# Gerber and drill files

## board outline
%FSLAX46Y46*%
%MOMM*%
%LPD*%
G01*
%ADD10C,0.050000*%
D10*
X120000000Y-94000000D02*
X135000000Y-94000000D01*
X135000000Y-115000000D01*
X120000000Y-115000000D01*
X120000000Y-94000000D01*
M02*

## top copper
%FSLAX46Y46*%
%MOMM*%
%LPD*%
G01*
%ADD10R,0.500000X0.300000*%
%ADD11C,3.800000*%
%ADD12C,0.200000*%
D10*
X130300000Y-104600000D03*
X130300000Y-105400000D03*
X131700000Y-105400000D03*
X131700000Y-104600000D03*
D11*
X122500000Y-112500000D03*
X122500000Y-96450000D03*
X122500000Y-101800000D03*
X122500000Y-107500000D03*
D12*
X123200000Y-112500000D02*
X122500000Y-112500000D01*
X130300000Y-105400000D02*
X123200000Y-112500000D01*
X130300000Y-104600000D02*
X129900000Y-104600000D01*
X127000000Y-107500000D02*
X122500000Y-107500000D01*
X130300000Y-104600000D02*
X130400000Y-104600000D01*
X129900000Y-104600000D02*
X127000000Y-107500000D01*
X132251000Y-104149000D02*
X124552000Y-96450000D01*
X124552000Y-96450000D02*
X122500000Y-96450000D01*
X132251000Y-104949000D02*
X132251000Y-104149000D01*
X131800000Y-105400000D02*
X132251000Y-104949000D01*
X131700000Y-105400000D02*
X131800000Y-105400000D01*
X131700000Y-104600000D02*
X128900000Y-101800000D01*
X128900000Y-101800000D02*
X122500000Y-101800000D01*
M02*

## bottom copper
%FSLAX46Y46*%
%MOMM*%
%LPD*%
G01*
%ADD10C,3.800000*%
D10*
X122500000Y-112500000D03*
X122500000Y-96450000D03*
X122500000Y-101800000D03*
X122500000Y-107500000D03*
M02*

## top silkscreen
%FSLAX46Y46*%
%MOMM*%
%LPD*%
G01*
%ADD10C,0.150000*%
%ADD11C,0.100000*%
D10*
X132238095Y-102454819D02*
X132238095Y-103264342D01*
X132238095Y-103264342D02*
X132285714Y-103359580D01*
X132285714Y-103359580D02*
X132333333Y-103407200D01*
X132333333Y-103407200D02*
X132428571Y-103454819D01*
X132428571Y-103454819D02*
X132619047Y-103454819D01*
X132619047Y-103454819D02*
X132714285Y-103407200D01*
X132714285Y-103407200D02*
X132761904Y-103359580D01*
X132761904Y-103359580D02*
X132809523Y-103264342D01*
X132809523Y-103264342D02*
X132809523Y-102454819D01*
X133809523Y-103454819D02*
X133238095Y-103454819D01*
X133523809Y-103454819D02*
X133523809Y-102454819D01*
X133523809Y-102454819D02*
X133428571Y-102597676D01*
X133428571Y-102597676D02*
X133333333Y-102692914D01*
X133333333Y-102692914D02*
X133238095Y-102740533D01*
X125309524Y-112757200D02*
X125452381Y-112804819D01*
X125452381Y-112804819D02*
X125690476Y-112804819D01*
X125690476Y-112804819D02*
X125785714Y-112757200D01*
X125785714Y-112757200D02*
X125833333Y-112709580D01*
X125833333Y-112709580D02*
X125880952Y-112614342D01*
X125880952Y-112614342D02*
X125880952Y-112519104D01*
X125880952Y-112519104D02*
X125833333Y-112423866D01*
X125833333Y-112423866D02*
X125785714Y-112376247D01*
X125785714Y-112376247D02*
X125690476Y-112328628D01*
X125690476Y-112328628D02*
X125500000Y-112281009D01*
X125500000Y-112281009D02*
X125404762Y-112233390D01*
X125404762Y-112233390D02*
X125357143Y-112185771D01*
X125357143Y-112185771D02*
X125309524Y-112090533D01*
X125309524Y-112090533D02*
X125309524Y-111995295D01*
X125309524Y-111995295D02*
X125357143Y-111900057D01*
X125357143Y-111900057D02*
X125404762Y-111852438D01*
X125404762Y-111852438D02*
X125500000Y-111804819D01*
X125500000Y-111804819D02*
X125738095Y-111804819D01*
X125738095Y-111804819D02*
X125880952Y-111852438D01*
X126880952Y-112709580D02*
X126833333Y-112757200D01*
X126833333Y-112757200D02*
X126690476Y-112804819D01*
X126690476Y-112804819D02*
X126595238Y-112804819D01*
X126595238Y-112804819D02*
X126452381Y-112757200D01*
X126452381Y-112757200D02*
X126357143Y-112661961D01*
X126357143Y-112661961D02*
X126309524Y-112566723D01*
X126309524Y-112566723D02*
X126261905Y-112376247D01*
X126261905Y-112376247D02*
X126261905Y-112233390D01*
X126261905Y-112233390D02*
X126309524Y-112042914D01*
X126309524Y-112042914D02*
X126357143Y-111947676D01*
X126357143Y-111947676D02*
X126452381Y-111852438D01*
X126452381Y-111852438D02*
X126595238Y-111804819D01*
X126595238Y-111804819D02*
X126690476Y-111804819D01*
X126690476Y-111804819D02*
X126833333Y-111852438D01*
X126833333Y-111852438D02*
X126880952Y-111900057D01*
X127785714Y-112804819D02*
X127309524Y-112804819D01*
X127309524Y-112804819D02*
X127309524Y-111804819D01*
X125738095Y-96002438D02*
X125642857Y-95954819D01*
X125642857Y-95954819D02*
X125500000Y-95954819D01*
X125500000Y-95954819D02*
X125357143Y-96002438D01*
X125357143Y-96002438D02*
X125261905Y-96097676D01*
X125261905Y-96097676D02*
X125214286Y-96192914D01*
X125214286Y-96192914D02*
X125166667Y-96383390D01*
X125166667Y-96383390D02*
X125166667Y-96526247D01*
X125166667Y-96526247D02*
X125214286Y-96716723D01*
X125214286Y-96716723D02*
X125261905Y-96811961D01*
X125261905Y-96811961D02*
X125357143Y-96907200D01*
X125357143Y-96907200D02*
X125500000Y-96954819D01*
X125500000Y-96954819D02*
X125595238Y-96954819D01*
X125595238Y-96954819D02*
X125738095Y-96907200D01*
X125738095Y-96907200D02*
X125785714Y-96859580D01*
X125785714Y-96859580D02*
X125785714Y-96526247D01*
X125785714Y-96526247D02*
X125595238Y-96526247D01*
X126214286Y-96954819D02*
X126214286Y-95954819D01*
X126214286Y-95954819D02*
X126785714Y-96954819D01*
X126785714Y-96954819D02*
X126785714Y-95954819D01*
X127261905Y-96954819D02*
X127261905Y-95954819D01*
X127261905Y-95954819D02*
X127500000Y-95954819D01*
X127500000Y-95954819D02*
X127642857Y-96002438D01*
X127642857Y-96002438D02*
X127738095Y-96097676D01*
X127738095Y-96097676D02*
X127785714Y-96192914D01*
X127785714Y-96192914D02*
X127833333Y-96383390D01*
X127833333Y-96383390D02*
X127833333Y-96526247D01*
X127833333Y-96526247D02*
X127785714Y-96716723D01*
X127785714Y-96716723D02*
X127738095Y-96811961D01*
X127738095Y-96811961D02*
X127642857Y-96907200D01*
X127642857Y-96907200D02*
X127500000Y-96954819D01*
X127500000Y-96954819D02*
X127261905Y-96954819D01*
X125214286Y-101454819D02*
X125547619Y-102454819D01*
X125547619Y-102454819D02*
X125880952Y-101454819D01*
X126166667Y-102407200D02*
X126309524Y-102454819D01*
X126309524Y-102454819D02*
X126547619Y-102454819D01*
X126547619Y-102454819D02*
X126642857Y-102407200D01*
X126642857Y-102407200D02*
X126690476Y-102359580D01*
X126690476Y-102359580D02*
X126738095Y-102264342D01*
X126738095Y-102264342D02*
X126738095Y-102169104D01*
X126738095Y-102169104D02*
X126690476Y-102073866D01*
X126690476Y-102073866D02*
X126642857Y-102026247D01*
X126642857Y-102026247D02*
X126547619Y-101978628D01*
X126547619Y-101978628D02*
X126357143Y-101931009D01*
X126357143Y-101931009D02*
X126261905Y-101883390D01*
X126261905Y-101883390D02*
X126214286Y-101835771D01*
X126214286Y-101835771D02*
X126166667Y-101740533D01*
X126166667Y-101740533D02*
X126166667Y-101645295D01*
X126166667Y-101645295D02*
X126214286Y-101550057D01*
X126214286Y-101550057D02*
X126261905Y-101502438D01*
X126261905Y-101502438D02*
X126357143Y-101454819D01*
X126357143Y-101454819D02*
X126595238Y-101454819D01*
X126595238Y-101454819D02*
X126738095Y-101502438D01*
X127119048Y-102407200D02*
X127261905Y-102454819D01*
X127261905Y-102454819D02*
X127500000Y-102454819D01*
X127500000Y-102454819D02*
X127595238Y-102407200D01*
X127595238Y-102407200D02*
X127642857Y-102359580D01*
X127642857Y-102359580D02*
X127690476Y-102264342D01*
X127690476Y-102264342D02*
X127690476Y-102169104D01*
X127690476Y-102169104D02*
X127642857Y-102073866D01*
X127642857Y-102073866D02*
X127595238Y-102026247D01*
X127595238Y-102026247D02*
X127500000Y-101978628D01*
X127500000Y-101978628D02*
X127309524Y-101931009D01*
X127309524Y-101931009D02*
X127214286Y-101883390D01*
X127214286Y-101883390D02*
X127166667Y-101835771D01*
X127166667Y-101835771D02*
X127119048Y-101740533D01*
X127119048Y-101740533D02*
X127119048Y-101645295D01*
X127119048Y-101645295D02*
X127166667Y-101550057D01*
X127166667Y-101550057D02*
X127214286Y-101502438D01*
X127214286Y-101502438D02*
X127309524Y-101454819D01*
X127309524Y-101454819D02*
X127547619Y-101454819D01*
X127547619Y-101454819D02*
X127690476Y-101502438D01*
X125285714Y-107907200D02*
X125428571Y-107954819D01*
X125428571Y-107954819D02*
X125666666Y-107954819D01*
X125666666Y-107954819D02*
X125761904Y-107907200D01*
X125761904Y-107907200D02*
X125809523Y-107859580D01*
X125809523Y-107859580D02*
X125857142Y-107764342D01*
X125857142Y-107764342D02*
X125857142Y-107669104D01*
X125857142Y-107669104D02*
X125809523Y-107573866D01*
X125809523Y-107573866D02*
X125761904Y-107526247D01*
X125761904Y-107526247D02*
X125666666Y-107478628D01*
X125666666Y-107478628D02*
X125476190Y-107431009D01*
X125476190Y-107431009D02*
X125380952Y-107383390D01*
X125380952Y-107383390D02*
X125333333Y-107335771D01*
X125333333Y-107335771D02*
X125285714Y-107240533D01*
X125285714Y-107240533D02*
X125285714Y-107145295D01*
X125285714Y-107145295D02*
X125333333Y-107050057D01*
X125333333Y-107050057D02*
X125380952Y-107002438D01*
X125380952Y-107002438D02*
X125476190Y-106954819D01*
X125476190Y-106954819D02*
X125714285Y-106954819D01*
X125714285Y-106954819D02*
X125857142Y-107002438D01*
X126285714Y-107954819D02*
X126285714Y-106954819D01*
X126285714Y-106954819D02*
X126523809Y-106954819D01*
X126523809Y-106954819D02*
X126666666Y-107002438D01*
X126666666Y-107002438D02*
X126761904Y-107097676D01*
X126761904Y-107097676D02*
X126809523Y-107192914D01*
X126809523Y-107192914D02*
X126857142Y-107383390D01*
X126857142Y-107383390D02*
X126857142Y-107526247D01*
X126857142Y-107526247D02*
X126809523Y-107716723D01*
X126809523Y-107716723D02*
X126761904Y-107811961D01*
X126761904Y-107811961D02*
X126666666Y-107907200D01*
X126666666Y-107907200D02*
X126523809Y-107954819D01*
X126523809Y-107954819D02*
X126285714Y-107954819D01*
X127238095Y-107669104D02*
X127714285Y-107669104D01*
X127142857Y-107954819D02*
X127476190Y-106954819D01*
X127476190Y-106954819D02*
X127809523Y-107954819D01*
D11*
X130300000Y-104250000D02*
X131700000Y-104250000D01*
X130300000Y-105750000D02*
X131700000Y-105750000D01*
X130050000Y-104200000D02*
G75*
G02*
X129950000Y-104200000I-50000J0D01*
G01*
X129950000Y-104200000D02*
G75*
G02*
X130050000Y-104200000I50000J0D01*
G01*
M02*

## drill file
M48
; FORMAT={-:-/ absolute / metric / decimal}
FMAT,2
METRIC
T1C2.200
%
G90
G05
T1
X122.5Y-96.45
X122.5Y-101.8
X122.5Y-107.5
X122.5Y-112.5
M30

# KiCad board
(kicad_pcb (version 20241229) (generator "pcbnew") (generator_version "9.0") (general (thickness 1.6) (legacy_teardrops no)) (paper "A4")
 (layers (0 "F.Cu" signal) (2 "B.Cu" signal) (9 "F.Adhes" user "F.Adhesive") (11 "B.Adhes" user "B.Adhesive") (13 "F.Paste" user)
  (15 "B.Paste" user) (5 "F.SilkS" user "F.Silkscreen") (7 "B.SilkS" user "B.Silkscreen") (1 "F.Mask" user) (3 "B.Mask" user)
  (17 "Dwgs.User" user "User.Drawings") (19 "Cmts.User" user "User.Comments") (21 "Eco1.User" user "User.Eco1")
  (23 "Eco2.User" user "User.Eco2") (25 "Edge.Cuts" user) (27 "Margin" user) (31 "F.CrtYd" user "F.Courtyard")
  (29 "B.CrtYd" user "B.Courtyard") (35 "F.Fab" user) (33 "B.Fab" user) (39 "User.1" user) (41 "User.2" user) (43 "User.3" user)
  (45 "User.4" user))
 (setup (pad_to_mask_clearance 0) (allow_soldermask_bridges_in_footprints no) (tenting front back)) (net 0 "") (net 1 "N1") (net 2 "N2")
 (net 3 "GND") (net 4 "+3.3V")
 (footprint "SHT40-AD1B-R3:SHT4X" (layer "F.Cu") (at 131 105)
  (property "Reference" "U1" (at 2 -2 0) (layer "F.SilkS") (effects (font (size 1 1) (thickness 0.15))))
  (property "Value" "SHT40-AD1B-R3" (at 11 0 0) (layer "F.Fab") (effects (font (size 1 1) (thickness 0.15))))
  (fp_line (start -0.7 -0.75) (end 0.7 -0.75) (stroke (width 0.1) (type solid)) (layer "F.SilkS"))
  (fp_line (start -0.7 0.75) (end 0.7 0.75) (stroke (width 0.1) (type solid)) (layer "F.SilkS"))
  (fp_circle (center -1 -0.8) (end -0.95 -0.8) (stroke (width 0.1) (type solid)) (fill no) (layer "F.SilkS"))
  (pad "1" smd rect (at -0.7 -0.4) (size 0.5 0.3) (layers "F.Cu" "F.Mask" "F.Paste") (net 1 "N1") (solder_mask_margin 0.102))
  (pad "2" smd rect (at -0.7 0.4) (size 0.5 0.3) (layers "F.Cu" "F.Mask" "F.Paste") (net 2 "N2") (solder_mask_margin 0.102))
  (pad "3" smd rect (at 0.7 0.4) (size 0.5 0.3) (layers "F.Cu" "F.Mask" "F.Paste") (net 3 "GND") (solder_mask_margin 0.102))
  (pad "4" smd rect (at 0.7 -0.4) (size 0.5 0.3) (layers "F.Cu" "F.Mask" "F.Paste") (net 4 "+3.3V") (solder_mask_margin 0.102)))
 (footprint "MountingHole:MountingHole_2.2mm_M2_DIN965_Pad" (layer "F.Cu") (at 122.5 112.5)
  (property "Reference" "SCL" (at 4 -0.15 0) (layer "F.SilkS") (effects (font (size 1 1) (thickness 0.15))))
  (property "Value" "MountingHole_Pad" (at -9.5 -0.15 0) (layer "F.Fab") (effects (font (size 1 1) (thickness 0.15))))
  (pad "1" thru_hole circle (at 0 0) (size 3.8 3.8) (drill 2.2) (layers "*.Cu" "*.Mask") (remove_unused_layers no) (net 2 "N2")
   (zone_connect 2)))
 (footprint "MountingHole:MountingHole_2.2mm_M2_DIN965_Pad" (layer "F.Cu") (at 122.5 96.45)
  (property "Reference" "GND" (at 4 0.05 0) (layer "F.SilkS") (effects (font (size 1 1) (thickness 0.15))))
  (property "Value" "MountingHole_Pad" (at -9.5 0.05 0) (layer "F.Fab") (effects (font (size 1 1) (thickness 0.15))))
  (pad "1" thru_hole circle (at 0 0) (size 3.8 3.8) (drill 2.2) (layers "*.Cu" "*.Mask") (remove_unused_layers no) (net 3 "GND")
   (zone_connect 2)))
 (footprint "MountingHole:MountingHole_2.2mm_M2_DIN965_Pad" (layer "F.Cu") (at 122.5 101.8)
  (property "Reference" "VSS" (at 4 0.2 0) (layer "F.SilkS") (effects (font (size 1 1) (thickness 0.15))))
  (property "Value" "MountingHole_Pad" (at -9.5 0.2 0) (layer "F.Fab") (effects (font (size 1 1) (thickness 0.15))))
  (pad "1" thru_hole circle (at 0 0) (size 3.8 3.8) (drill 2.2) (layers "*.Cu" "*.Mask") (remove_unused_layers no) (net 4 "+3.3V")
   (zone_connect 2)))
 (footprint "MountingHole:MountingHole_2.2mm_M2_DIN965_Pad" (layer "F.Cu") (at 122.5 107.5)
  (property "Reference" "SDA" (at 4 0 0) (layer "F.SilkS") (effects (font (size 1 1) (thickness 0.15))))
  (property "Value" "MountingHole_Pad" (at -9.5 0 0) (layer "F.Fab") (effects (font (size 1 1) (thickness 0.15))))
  (pad "1" thru_hole circle (at 0 0) (size 3.8 3.8) (drill 2.2) (layers "*.Cu" "*.Mask") (remove_unused_layers no) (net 1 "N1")
   (zone_connect 2)))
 (gr_rect (start 120 94) (end 135 115) (stroke (width 0.05) (type default)) (fill no) (layer "Edge.Cuts"))
 (segment (start 123.2 112.5) (end 122.5 112.5) (width 0.2) (layer "F.Cu") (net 2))
 (segment (start 130.3 105.4) (end 123.2 112.5) (width 0.2) (layer "F.Cu") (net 2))
 (segment (start 130.3 104.6) (end 129.9 104.6) (width 0.2) (layer "F.Cu") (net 1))
 (segment (start 127 107.5) (end 122.5 107.5) (width 0.2) (layer "F.Cu") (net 1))
 (segment (start 130.3 104.6) (end 130.4 104.6) (width 0.2) (layer "F.Cu") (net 1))
 (segment (start 129.9 104.6) (end 127 107.5) (width 0.2) (layer "F.Cu") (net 1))
 (segment (start 132.251 104.149) (end 124.552 96.45) (width 0.2) (layer "F.Cu") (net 3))
 (segment (start 124.552 96.45) (end 122.5 96.45) (width 0.2) (layer "F.Cu") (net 3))
 (segment (start 132.251 104.949) (end 132.251 104.149) (width 0.2) (layer "F.Cu") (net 3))
 (segment (start 131.8 105.4) (end 132.251 104.949) (width 0.2) (layer "F.Cu") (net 3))
 (segment (start 131.7 105.4) (end 131.8 105.4) (width 0.2) (layer "F.Cu") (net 3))
 (segment (start 131.7 104.6) (end 128.9 101.8) (width 0.2) (layer "F.Cu") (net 4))
 (segment (start 128.9 101.8) (end 122.5 101.8) (width 0.2) (layer "F.Cu") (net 4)))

